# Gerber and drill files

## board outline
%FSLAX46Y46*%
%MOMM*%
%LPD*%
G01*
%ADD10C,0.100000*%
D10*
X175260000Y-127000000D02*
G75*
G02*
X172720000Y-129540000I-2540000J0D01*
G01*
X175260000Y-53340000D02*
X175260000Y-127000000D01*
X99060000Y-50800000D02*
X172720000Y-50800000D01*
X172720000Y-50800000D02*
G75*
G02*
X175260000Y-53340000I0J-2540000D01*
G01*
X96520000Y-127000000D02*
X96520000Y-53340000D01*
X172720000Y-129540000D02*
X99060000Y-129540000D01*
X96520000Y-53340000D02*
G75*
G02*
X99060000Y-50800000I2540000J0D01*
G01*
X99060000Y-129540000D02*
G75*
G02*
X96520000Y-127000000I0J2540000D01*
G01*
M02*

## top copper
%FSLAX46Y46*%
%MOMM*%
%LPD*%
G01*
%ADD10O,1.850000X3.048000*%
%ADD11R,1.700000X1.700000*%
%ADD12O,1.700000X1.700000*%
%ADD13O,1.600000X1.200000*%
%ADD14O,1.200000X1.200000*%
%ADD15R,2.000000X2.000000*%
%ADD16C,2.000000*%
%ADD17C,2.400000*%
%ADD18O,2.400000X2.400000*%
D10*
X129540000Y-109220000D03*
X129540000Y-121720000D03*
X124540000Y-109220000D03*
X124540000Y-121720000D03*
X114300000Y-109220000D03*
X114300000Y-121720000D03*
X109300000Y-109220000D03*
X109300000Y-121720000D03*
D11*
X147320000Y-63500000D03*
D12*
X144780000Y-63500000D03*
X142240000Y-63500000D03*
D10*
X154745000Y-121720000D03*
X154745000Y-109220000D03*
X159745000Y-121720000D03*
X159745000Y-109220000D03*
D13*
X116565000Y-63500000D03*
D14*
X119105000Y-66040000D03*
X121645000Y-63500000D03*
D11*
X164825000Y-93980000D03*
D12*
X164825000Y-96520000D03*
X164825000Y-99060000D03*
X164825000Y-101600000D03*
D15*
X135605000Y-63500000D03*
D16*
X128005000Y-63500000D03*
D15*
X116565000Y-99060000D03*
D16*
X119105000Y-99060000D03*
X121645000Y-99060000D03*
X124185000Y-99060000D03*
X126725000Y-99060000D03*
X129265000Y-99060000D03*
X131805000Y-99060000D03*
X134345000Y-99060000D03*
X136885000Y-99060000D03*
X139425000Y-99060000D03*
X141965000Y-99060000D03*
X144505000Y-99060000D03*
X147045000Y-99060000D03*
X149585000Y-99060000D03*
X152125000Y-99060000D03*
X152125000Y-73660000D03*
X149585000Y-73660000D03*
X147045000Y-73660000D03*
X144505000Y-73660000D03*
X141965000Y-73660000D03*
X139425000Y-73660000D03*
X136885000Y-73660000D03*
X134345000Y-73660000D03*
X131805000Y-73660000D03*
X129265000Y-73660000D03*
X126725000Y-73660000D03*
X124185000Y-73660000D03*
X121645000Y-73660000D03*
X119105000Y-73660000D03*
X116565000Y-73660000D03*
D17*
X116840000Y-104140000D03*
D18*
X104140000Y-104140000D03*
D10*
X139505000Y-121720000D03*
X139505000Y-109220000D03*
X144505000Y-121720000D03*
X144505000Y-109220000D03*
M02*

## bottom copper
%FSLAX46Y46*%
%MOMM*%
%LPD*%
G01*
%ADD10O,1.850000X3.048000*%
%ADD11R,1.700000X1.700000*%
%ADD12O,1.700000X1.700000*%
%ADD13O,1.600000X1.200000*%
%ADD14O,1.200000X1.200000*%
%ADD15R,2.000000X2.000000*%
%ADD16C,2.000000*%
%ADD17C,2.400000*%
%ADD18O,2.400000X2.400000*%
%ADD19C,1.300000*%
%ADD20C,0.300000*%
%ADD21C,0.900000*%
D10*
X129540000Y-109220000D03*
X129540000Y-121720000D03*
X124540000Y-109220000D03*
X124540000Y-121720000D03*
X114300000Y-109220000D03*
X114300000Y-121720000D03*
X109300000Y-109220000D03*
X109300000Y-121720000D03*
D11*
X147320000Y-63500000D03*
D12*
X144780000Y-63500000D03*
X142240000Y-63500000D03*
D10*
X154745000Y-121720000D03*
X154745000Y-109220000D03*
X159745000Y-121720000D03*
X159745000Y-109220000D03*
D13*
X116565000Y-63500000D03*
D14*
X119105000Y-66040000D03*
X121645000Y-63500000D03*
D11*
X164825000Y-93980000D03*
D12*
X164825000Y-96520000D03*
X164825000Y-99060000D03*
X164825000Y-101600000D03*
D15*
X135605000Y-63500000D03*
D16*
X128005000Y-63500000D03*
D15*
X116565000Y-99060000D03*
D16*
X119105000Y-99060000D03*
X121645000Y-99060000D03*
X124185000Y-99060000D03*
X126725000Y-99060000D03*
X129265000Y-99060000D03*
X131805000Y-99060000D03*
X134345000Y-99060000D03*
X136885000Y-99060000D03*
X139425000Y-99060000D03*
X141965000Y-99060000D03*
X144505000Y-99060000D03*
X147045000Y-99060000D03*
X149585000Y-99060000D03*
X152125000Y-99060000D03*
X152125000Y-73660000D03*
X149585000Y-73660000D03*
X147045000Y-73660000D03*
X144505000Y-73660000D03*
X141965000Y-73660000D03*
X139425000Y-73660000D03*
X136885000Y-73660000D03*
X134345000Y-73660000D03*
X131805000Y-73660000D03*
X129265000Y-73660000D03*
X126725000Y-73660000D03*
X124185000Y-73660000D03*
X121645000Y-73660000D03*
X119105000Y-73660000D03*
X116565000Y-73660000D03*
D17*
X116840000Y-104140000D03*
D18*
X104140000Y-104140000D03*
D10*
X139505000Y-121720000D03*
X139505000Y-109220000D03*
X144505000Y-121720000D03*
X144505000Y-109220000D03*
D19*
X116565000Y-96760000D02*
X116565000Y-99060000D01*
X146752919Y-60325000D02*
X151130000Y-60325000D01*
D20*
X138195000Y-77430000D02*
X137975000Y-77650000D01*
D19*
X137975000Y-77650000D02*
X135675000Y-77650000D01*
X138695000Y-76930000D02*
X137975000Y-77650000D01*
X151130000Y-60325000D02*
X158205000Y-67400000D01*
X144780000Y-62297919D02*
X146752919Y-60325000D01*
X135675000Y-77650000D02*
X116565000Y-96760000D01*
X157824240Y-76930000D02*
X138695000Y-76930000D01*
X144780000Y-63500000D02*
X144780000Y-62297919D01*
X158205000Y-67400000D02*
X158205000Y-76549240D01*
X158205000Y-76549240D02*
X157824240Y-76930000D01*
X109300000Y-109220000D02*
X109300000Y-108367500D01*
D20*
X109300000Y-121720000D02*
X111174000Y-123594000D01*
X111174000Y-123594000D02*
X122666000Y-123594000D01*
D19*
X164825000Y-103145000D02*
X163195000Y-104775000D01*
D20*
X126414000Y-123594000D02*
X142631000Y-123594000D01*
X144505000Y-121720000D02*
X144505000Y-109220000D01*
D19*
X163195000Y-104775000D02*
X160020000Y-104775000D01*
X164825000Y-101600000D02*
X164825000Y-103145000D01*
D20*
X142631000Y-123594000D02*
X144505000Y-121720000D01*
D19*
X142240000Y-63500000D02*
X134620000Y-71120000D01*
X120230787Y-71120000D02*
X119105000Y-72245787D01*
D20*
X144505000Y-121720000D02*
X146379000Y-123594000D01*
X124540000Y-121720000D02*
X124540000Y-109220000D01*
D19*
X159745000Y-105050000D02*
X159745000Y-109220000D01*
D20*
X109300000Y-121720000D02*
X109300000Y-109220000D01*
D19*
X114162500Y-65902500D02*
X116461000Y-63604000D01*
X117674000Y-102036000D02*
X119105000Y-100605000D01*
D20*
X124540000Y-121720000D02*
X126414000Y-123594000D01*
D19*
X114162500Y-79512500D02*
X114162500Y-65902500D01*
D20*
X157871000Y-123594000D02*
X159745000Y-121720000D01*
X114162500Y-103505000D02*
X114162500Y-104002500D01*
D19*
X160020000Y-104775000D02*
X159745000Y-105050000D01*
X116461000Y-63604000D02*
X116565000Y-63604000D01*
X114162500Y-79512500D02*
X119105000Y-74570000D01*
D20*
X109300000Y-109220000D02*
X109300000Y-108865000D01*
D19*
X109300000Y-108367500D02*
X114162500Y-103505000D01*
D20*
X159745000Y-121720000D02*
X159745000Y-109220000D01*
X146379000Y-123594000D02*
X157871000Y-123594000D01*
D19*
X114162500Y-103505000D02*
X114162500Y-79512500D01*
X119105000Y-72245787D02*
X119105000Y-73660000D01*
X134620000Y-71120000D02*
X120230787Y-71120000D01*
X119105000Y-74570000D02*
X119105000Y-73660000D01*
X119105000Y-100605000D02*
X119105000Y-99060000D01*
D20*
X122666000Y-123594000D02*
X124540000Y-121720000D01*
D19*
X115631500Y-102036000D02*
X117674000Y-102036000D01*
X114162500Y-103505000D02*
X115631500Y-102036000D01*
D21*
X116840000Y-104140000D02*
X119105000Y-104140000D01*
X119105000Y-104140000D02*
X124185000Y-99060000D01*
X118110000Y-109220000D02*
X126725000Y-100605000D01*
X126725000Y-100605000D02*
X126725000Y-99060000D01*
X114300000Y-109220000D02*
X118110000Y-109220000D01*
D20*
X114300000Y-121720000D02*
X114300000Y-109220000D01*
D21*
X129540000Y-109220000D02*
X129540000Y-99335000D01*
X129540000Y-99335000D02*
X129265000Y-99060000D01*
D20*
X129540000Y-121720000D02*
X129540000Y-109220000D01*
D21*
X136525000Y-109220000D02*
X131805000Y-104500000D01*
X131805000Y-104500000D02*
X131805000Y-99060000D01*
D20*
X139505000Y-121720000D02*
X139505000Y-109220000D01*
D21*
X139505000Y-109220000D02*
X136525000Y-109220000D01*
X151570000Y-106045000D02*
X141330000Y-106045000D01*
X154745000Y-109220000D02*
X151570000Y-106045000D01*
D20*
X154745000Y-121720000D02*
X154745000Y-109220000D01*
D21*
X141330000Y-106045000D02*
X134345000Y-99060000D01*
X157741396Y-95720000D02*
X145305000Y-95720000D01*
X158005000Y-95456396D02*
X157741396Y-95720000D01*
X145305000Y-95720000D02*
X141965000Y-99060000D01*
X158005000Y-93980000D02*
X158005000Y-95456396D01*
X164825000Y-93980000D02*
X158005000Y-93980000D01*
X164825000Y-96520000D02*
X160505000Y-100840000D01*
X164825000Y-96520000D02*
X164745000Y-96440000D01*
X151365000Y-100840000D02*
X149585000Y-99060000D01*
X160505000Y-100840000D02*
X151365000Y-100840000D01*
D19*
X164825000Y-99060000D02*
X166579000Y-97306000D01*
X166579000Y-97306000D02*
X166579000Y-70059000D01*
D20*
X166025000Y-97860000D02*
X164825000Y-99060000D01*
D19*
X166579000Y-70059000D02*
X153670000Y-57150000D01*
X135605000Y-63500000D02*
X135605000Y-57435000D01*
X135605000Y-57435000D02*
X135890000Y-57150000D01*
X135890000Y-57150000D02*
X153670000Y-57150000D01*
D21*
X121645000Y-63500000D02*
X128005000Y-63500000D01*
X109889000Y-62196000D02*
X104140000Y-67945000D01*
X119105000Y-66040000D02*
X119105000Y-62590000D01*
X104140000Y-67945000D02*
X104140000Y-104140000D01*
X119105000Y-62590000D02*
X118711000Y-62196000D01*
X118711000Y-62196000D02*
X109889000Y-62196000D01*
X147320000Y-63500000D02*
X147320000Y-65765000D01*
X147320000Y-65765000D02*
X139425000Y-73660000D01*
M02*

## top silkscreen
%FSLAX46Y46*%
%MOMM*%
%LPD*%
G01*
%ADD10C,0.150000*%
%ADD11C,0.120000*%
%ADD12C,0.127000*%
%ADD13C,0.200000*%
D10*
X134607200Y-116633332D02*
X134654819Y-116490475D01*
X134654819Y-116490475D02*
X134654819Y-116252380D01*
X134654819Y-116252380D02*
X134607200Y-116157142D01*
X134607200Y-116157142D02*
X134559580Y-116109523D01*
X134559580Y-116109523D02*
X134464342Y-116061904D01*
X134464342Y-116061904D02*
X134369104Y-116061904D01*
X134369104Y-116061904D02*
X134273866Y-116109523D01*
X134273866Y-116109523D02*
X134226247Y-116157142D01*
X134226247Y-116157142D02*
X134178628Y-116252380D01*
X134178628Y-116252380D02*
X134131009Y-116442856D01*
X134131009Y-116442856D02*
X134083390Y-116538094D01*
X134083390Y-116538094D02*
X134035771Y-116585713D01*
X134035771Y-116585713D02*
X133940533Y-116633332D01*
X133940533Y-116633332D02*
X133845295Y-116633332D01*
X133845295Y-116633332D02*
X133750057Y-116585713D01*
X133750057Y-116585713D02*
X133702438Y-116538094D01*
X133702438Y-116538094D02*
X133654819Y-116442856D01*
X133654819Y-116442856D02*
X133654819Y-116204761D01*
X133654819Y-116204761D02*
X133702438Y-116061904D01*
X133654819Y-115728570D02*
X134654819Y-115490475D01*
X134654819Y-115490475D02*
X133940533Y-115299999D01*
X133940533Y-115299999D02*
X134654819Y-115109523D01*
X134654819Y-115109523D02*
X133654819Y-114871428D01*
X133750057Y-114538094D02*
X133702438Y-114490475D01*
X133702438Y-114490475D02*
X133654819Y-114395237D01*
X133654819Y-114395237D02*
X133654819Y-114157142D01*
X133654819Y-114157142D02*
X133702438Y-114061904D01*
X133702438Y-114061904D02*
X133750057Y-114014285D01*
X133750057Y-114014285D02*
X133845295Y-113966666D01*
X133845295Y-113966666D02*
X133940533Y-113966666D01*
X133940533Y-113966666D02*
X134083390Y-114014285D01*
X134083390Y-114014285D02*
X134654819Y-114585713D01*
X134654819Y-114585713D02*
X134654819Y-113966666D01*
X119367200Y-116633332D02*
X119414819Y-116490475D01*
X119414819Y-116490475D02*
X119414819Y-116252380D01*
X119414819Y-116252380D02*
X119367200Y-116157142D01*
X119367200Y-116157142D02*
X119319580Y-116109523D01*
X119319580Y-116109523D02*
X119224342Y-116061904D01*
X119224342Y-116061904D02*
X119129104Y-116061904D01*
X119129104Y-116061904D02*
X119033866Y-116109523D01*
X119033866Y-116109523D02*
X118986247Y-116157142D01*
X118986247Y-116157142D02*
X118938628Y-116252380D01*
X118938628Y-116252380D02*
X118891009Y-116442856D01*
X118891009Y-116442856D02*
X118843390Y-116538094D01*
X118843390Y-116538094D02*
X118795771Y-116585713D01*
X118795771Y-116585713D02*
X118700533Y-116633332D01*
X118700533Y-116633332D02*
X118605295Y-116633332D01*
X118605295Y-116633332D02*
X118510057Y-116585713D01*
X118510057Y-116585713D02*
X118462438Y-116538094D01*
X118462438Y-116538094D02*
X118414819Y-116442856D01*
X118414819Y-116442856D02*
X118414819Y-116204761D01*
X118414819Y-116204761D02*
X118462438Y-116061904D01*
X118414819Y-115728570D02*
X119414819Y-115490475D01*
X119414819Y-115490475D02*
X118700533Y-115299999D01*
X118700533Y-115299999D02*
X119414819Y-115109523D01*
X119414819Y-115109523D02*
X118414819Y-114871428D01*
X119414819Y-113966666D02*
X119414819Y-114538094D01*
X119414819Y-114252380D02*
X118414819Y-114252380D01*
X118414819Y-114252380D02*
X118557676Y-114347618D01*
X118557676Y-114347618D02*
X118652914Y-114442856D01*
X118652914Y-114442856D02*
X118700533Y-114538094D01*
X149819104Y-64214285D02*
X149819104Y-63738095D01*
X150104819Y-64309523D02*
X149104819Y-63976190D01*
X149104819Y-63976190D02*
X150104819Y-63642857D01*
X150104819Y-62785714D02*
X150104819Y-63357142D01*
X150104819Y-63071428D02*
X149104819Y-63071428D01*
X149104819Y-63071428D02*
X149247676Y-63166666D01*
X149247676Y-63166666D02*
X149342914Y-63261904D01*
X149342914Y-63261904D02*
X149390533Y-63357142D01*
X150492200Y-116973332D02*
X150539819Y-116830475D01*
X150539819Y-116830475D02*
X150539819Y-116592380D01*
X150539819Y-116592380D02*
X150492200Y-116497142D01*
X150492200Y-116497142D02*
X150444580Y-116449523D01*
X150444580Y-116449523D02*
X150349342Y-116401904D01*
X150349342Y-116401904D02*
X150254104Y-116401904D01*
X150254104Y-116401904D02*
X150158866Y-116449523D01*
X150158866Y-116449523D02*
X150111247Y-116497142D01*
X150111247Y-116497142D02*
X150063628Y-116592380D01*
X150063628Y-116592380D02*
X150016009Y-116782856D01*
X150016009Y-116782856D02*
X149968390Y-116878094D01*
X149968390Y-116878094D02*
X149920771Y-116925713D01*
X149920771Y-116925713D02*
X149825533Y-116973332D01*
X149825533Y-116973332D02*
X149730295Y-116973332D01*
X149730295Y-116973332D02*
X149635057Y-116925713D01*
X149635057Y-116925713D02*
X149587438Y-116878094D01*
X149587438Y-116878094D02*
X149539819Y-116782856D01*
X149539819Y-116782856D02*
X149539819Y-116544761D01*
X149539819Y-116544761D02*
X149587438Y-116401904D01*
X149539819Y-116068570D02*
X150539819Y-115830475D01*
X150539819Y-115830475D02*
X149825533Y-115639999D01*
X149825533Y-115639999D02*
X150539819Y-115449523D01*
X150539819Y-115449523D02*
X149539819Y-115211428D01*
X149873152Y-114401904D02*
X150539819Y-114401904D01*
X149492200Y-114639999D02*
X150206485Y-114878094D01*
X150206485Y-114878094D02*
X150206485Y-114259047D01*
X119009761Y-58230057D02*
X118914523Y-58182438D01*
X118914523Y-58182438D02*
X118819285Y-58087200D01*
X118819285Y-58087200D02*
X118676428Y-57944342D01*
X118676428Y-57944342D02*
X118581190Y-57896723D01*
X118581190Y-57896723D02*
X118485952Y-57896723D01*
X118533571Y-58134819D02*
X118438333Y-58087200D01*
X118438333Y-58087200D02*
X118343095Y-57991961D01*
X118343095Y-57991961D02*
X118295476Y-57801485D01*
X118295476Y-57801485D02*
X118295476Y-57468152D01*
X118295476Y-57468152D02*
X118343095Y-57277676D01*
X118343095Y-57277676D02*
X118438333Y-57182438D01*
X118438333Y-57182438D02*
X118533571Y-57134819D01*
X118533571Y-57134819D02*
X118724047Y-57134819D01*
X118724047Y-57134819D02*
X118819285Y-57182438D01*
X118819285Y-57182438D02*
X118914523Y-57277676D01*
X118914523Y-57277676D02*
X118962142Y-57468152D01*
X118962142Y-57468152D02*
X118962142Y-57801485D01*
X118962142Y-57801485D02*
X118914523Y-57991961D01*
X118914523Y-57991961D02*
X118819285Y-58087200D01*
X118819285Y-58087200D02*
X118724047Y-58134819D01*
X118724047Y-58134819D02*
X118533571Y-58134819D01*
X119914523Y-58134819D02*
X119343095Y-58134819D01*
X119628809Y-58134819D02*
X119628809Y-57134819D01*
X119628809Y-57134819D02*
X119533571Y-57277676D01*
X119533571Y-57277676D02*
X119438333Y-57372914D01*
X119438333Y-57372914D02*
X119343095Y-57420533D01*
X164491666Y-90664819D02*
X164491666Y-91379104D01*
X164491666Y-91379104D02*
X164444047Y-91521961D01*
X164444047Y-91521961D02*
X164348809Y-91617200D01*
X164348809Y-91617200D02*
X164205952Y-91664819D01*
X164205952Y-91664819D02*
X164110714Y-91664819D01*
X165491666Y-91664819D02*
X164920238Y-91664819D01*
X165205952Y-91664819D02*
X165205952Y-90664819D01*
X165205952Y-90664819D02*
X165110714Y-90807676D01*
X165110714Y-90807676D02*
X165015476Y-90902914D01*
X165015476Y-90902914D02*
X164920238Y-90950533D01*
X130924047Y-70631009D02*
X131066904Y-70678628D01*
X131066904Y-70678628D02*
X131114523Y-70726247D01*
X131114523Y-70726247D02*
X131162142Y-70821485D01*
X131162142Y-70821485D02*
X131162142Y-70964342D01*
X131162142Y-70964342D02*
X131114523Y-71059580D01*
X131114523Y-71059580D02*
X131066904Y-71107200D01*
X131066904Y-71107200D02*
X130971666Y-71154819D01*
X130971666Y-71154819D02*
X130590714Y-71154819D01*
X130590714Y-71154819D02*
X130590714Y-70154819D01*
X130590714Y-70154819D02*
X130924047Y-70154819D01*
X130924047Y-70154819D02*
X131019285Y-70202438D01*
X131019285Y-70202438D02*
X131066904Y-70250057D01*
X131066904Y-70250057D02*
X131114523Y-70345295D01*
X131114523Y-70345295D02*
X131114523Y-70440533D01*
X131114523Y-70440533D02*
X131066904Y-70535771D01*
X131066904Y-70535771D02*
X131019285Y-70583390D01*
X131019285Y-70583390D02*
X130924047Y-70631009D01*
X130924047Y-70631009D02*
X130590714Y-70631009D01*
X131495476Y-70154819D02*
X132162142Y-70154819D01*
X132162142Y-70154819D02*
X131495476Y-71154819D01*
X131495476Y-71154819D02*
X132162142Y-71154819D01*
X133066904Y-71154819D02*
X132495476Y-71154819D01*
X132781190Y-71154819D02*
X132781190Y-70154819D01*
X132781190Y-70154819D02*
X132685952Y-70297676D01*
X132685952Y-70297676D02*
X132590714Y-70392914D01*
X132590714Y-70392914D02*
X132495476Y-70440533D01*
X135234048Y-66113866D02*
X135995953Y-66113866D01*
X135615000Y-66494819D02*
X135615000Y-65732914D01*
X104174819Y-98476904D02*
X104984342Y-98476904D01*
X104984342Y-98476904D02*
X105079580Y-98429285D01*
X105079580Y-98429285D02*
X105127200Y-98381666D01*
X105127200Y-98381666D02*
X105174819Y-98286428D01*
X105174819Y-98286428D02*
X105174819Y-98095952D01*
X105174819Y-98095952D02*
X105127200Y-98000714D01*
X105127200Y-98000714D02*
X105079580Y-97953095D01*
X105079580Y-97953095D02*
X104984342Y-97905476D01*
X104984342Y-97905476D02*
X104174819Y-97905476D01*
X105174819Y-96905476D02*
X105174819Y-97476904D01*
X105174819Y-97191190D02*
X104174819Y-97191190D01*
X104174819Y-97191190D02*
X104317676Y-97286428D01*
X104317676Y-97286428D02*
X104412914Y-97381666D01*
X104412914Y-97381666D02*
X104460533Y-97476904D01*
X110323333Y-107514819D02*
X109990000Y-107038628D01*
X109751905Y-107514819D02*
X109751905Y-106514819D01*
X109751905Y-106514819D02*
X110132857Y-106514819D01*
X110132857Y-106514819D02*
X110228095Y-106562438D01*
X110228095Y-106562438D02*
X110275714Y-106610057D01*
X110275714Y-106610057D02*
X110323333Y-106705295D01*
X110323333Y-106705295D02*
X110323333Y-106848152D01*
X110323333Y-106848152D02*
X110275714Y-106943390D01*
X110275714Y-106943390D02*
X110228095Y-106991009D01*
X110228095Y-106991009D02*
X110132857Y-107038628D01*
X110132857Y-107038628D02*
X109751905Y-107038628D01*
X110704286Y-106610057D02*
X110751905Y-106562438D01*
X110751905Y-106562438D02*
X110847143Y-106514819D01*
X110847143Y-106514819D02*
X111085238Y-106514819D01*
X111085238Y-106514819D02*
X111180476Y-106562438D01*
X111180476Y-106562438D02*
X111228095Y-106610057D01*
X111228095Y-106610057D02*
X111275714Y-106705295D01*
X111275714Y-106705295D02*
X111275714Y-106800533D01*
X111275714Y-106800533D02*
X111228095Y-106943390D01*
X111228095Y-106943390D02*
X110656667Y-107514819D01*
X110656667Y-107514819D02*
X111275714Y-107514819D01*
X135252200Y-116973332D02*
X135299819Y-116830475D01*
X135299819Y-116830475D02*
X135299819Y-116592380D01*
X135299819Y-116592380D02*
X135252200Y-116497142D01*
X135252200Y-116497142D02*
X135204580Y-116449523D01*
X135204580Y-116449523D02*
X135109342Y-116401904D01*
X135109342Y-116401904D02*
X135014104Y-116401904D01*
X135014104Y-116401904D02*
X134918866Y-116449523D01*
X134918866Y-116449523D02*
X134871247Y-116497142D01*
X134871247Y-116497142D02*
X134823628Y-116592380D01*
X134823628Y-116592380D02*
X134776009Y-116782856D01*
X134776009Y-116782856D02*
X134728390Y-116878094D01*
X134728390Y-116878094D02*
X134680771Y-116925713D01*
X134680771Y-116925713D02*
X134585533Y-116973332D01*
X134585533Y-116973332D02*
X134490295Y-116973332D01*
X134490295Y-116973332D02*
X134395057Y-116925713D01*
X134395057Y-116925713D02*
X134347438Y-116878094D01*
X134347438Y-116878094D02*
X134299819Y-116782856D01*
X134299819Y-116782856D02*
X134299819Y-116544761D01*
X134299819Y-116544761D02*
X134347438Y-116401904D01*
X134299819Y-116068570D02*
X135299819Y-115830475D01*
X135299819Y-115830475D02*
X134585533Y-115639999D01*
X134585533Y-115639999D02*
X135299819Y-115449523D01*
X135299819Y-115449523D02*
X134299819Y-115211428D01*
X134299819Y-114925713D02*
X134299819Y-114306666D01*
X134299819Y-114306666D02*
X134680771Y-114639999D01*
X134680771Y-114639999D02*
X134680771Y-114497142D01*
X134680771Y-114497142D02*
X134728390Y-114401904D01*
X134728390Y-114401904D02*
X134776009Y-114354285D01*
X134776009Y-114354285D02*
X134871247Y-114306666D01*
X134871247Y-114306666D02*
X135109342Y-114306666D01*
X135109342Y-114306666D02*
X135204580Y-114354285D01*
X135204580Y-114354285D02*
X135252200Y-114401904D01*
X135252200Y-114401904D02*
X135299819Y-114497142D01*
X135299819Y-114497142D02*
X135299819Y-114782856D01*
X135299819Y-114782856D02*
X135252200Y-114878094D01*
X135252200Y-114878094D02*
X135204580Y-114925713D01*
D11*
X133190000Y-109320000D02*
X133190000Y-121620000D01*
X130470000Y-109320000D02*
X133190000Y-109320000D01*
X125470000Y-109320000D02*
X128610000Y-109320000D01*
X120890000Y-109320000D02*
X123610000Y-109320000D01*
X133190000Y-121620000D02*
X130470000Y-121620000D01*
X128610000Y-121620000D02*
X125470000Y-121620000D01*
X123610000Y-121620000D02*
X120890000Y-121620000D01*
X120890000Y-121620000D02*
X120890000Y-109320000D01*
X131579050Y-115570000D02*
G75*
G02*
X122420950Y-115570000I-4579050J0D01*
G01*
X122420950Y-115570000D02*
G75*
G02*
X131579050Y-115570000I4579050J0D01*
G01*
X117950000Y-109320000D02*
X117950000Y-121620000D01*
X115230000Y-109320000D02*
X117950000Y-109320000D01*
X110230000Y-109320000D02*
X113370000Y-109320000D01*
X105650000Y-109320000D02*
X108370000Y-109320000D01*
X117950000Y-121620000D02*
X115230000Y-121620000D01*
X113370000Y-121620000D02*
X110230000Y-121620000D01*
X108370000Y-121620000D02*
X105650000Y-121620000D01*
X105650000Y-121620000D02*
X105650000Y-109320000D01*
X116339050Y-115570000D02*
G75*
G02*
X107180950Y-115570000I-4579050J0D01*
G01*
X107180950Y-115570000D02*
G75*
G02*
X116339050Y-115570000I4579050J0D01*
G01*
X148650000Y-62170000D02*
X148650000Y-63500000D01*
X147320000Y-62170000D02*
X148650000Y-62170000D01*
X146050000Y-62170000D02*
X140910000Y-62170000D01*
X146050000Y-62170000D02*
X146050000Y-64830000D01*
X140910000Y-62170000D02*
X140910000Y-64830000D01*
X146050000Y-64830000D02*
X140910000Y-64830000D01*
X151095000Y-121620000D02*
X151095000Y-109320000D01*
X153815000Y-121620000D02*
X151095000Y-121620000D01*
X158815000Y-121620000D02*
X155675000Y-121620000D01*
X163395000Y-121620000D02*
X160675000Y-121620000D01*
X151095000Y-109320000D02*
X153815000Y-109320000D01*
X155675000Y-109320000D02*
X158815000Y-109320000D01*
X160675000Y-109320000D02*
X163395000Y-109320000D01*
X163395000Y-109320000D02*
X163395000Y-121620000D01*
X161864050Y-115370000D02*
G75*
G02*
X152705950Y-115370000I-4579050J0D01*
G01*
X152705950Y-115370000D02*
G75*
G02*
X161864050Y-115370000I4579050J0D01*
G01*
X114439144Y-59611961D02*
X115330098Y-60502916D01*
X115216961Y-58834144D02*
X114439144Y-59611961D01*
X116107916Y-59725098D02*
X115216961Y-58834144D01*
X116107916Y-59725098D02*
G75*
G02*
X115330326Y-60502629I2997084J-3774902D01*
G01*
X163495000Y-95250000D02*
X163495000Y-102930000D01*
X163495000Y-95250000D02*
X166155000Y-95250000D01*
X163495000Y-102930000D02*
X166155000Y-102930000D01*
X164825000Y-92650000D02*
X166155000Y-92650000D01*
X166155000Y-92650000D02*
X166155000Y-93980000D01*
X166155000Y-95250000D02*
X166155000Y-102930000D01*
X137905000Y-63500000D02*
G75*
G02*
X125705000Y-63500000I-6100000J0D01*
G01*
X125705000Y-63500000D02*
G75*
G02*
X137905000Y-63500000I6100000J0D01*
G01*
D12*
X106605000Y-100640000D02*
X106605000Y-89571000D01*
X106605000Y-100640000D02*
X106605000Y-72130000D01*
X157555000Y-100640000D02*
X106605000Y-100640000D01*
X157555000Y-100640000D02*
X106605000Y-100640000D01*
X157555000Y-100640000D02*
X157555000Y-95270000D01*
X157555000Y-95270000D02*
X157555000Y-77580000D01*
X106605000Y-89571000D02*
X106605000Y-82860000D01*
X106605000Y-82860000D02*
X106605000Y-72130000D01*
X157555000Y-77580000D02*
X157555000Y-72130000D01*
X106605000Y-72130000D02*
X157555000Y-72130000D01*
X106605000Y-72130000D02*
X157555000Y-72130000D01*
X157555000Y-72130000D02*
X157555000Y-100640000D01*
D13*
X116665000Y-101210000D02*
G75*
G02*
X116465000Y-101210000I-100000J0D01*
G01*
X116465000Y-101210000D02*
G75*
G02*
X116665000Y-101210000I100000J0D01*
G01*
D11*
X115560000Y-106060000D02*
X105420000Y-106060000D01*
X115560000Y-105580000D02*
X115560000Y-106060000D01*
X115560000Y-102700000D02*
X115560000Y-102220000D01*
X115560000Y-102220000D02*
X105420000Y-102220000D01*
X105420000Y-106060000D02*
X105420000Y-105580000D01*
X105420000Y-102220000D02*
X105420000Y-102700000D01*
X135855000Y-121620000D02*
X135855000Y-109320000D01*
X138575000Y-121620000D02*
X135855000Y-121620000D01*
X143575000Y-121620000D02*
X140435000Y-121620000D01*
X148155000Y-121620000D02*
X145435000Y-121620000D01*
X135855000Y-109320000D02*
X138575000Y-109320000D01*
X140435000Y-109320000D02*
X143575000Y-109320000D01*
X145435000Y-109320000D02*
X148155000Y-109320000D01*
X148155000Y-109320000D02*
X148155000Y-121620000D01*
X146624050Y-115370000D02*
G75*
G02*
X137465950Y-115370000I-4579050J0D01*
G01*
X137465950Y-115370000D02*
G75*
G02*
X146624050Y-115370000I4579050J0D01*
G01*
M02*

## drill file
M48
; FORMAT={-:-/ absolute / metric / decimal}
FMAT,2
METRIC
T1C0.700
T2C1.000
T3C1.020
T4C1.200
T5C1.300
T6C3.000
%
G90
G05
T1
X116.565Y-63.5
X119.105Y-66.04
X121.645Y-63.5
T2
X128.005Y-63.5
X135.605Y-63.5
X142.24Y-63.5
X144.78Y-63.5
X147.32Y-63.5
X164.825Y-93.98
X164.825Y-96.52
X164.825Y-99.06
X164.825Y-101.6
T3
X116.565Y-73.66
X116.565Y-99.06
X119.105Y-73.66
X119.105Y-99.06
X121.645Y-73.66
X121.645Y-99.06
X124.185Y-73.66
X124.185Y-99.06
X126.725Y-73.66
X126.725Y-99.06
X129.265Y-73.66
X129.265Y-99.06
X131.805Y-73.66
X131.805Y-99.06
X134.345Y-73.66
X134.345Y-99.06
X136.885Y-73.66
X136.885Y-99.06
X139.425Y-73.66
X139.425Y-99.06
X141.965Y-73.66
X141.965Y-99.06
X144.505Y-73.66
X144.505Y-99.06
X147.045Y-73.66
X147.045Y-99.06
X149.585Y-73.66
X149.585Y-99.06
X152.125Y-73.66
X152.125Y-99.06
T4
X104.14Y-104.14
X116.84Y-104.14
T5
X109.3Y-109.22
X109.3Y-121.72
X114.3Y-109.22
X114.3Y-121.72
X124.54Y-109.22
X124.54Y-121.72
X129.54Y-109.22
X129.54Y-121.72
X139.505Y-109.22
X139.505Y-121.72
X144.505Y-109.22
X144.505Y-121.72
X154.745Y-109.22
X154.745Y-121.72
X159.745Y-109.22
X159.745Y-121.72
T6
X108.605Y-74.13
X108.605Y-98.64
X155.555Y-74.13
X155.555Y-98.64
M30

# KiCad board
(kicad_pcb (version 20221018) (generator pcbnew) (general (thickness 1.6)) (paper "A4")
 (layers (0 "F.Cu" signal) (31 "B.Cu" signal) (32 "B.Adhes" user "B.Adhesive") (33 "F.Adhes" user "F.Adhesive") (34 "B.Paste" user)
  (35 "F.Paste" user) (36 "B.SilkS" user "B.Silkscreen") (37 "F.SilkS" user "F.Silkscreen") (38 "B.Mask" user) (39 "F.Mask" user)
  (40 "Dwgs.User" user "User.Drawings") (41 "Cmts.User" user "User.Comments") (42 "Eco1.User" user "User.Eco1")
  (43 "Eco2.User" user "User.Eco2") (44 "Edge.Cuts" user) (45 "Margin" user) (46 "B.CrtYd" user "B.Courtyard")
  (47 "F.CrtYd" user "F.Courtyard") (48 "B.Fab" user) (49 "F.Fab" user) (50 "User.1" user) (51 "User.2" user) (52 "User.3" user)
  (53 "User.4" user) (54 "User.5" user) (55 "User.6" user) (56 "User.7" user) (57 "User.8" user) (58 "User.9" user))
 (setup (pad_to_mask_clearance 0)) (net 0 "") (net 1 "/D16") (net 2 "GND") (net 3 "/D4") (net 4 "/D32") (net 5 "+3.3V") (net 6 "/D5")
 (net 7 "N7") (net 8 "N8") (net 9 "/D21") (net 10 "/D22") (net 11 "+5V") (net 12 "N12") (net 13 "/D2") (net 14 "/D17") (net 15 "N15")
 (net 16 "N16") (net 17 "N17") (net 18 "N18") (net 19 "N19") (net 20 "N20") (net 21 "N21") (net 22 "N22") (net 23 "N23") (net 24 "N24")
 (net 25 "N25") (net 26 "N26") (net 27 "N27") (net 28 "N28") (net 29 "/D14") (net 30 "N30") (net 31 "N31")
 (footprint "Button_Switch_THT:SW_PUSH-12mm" (layer "F.Cu") (at 129.54 109.22 -90)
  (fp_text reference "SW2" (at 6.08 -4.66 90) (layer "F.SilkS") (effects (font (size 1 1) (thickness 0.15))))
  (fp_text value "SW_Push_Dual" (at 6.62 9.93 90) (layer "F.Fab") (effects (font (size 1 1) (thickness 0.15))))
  (fp_line (start 0.1 -3.65) (end 12.4 -3.65) (stroke (width 0.12) (type solid)) (layer "F.SilkS"))
  (fp_line (start 0.1 -0.93) (end 0.1 -3.65) (stroke (width 0.12) (type solid)) (layer "F.SilkS"))
  (fp_line (start 0.1 4.07) (end 0.1 0.93) (stroke (width 0.12) (type solid)) (layer "F.SilkS"))
  (fp_line (start 0.1 8.65) (end 0.1 5.93) (stroke (width 0.12) (type solid)) (layer "F.SilkS"))
  (fp_line (start 12.4 -3.65) (end 12.4 -0.93) (stroke (width 0.12) (type solid)) (layer "F.SilkS"))
  (fp_line (start 12.4 0.93) (end 12.4 4.07) (stroke (width 0.12) (type solid)) (layer "F.SilkS"))
  (fp_line (start 12.4 5.93) (end 12.4 8.65) (stroke (width 0.12) (type solid)) (layer "F.SilkS"))
  (fp_line (start 12.4 8.65) (end 0.1 8.65) (stroke (width 0.12) (type solid)) (layer "F.SilkS"))
  (fp_circle (center 6.35 2.54) (end 10.16 5.08) (stroke (width 0.12) (type solid)) (fill none) (layer "F.SilkS"))
  (pad "1" thru_hole oval (at 0 0 270) (size 3.048 1.85) (drill 1.3) (layers "*.Cu" "*.Mask") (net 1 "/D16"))
  (pad "1" thru_hole oval (at 12.5 0 270) (size 3.048 1.85) (drill 1.3) (layers "*.Cu" "*.Mask") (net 1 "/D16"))
  (pad "2" thru_hole oval (at 0 5 270) (size 3.048 1.85) (drill 1.3) (layers "*.Cu" "*.Mask") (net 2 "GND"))
  (pad "2" thru_hole oval (at 12.5 5 270) (size 3.048 1.85) (drill 1.3) (layers "*.Cu" "*.Mask") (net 2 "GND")))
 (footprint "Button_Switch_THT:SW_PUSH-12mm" (layer "F.Cu") (at 114.3 109.22 -90)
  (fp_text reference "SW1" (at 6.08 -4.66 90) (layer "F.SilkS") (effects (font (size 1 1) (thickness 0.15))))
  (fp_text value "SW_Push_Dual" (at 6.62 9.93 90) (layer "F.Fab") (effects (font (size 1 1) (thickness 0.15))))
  (fp_line (start 0.1 -3.65) (end 12.4 -3.65) (stroke (width 0.12) (type solid)) (layer "F.SilkS"))
  (fp_line (start 0.1 -0.93) (end 0.1 -3.65) (stroke (width 0.12) (type solid)) (layer "F.SilkS"))
  (fp_line (start 0.1 4.07) (end 0.1 0.93) (stroke (width 0.12) (type solid)) (layer "F.SilkS"))
  (fp_line (start 0.1 8.65) (end 0.1 5.93) (stroke (width 0.12) (type solid)) (layer "F.SilkS"))
  (fp_line (start 12.4 -3.65) (end 12.4 -0.93) (stroke (width 0.12) (type solid)) (layer "F.SilkS"))
  (fp_line (start 12.4 0.93) (end 12.4 4.07) (stroke (width 0.12) (type solid)) (layer "F.SilkS"))
  (fp_line (start 12.4 5.93) (end 12.4 8.65) (stroke (width 0.12) (type solid)) (layer "F.SilkS"))
  (fp_line (start 12.4 8.65) (end 0.1 8.65) (stroke (width 0.12) (type solid)) (layer "F.SilkS"))
  (fp_circle (center 6.35 2.54) (end 10.16 5.08) (stroke (width 0.12) (type solid)) (fill none) (layer "F.SilkS"))
  (pad "1" thru_hole oval (at 0 0 270) (size 3.048 1.85) (drill 1.3) (layers "*.Cu" "*.Mask") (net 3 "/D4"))
  (pad "1" thru_hole oval (at 12.5 0 270) (size 3.048 1.85) (drill 1.3) (layers "*.Cu" "*.Mask") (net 3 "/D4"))
  (pad "2" thru_hole oval (at 0 5 270) (size 3.048 1.85) (drill 1.3) (layers "*.Cu" "*.Mask") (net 2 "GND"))
  (pad "2" thru_hole oval (at 12.5 5 270) (size 3.048 1.85) (drill 1.3) (layers "*.Cu" "*.Mask") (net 2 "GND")))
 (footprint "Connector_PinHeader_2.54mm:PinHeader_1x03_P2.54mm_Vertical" (layer "F.Cu") (at 147.32 63.5 -90)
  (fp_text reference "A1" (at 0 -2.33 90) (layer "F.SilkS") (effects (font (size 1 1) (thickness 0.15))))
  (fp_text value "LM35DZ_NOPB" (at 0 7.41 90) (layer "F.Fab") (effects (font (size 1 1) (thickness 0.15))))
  (fp_line (start -1.33 -1.33) (end 0 -1.33) (stroke (width 0.12) (type solid)) (layer "F.SilkS"))
  (fp_line (start -1.33 0) (end -1.33 -1.33) (stroke (width 0.12) (type solid)) (layer "F.SilkS"))
  (fp_line (start -1.33 1.27) (end -1.33 6.41) (stroke (width 0.12) (type solid)) (layer "F.SilkS"))
  (fp_line (start -1.33 1.27) (end 1.33 1.27) (stroke (width 0.12) (type solid)) (layer "F.SilkS"))
  (fp_line (start -1.33 6.41) (end 1.33 6.41) (stroke (width 0.12) (type solid)) (layer "F.SilkS"))
  (fp_line (start 1.33 1.27) (end 1.33 6.41) (stroke (width 0.12) (type solid)) (layer "F.SilkS"))
  (pad "1" thru_hole rect (at 0 0 270) (size 1.7 1.7) (drill 1) (layers "*.Cu" "*.Mask") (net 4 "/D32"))
  (pad "2" thru_hole oval (at 0 2.54 270) (size 1.7 1.7) (drill 1) (layers "*.Cu" "*.Mask") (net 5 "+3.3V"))
  (pad "3" thru_hole oval (at 0 5.08 270) (size 1.7 1.7) (drill 1) (layers "*.Cu" "*.Mask") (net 2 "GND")))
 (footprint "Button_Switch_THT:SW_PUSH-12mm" (layer "F.Cu") (at 154.745 121.72 90)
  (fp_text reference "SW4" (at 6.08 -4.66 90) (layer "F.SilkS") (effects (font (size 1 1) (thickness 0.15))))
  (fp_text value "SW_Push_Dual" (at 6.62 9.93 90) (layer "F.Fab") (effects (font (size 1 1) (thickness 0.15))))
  (fp_line (start 0.1 -3.65) (end 12.4 -3.65) (stroke (width 0.12) (type solid)) (layer "F.SilkS"))
  (fp_line (start 0.1 -0.93) (end 0.1 -3.65) (stroke (width 0.12) (type solid)) (layer "F.SilkS"))
  (fp_line (start 0.1 4.07) (end 0.1 0.93) (stroke (width 0.12) (type solid)) (layer "F.SilkS"))
  (fp_line (start 0.1 8.65) (end 0.1 5.93) (stroke (width 0.12) (type solid)) (layer "F.SilkS"))
  (fp_line (start 12.4 -3.65) (end 12.4 -0.93) (stroke (width 0.12) (type solid)) (layer "F.SilkS"))
  (fp_line (start 12.4 0.93) (end 12.4 4.07) (stroke (width 0.12) (type solid)) (layer "F.SilkS"))
  (fp_line (start 12.4 5.93) (end 12.4 8.65) (stroke (width 0.12) (type solid)) (layer "F.SilkS"))
  (fp_line (start 12.4 8.65) (end 0.1 8.65) (stroke (width 0.12) (type solid)) (layer "F.SilkS"))
  (fp_circle (center 6.35 2.54) (end 10.16 5.08) (stroke (width 0.12) (type solid)) (fill none) (layer "F.SilkS"))
  (pad "1" thru_hole oval (at 0 0 90) (size 3.048 1.85) (drill 1.3) (layers "*.Cu" "*.Mask") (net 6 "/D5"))
  (pad "1" thru_hole oval (at 12.5 0 90) (size 3.048 1.85) (drill 1.3) (layers "*.Cu" "*.Mask") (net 6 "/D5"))
  (pad "2" thru_hole oval (at 0 5 90) (size 3.048 1.85) (drill 1.3) (layers "*.Cu" "*.Mask") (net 2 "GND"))
  (pad "2" thru_hole oval (at 12.5 5 90) (size 3.048 1.85) (drill 1.3) (layers "*.Cu" "*.Mask") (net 2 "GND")))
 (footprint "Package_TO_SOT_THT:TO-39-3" (layer "F.Cu") (at 116.565 63.5)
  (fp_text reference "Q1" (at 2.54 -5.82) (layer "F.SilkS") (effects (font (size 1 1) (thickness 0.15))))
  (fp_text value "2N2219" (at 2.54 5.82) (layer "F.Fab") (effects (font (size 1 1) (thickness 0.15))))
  (fp_line (start -2.125856 -3.888039) (end -1.234902 -2.997084) (stroke (width 0.12) (type solid)) (layer "F.SilkS"))
  (fp_line (start -1.348039 -4.665856) (end -2.125856 -3.888039) (stroke (width 0.12) (type solid)) (layer "F.SilkS"))
  (fp_line (start -0.457084 -3.774902) (end -1.348039 -4.665856) (stroke (width 0.12) (type solid)) (layer "F.SilkS"))
  (fp_arc (start -0.457084 -3.774902) (mid 5.948125 3.408384) (end -1.234674 -2.997371) (stroke (width 0.12) (type solid)) (layer "F.SilkS"))
  (pad "1" thru_hole oval (at 0 0) (size 1.6 1.2) (drill 0.7) (layers "*.Cu" "*.Mask") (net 2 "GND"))
  (pad "2" thru_hole oval (at 2.54 2.54) (size 1.2 1.2) (drill 0.7) (layers "*.Cu" "*.Mask") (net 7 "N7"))
  (pad "3" thru_hole oval (at 5.08 0) (size 1.2 1.2) (drill 0.7) (layers "*.Cu" "*.Mask") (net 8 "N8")))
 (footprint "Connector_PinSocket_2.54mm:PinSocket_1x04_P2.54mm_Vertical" (layer "F.Cu") (at 164.825 93.98)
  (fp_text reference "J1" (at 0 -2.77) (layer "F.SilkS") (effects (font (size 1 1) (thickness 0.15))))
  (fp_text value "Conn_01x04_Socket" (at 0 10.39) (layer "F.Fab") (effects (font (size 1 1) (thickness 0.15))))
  (fp_line (start -1.33 1.27) (end -1.33 8.95) (stroke (width 0.12) (type solid)) (layer "F.SilkS"))
  (fp_line (start -1.33 1.27) (end 1.33 1.27) (stroke (width 0.12) (type solid)) (layer "F.SilkS"))
  (fp_line (start -1.33 8.95) (end 1.33 8.95) (stroke (width 0.12) (type solid)) (layer "F.SilkS"))
  (fp_line (start 0 -1.33) (end 1.33 -1.33) (stroke (width 0.12) (type solid)) (layer "F.SilkS"))
  (fp_line (start 1.33 -1.33) (end 1.33 0) (stroke (width 0.12) (type solid)) (layer "F.SilkS"))
  (fp_line (start 1.33 1.27) (end 1.33 8.95) (stroke (width 0.12) (type solid)) (layer "F.SilkS"))
  (pad "1" thru_hole rect (at 0 0) (size 1.7 1.7) (drill 1) (layers "*.Cu" "*.Mask") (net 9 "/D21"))
  (pad "2" thru_hole oval (at 0 2.54) (size 1.7 1.7) (drill 1) (layers "*.Cu" "*.Mask") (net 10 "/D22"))
  (pad "3" thru_hole oval (at 0 5.08) (size 1.7 1.7) (drill 1) (layers "*.Cu" "*.Mask") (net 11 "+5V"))
  (pad "4" thru_hole oval (at 0 7.62) (size 1.7 1.7) (drill 1) (layers "*.Cu" "*.Mask") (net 2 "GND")))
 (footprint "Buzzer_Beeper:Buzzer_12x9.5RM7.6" (layer "F.Cu") (at 135.605 63.5 180)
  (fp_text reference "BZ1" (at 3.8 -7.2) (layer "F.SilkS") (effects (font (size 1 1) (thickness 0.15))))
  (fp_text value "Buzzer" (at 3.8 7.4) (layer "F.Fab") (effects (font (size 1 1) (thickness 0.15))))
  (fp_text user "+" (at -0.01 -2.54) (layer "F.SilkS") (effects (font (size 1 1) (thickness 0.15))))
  (fp_circle (center 3.8 0) (end 9.9 0) (stroke (width 0.12) (type solid)) (fill none) (layer "F.SilkS"))
  (pad "1" thru_hole rect (at 0 0 180) (size 2 2) (drill 1) (layers "*.Cu" "*.Mask") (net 11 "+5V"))
  (pad "2" thru_hole circle (at 7.6 0 180) (size 2 2) (drill 1) (layers "*.Cu" "*.Mask") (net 8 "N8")))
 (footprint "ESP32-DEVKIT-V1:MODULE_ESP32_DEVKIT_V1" (layer "F.Cu") (at 132.08 86.36 90)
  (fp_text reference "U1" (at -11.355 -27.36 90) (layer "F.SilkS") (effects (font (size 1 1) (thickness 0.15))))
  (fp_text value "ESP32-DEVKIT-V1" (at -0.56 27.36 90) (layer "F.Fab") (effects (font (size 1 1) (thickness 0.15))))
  (fp_line (start -14.28 -25.475) (end -3.211 -25.475) (stroke (width 0.127) (type solid)) (layer "F.SilkS"))
  (fp_line (start -14.28 -25.475) (end 14.23 -25.475) (stroke (width 0.127) (type solid)) (layer "F.SilkS"))
  (fp_line (start -14.28 25.475) (end -14.28 -25.475) (stroke (width 0.127) (type solid)) (layer "F.SilkS"))
  (fp_line (start -14.28 25.475) (end -14.28 -25.475) (stroke (width 0.127) (type solid)) (layer "F.SilkS"))
  (fp_line (start -14.28 25.475) (end -8.91 25.475) (stroke (width 0.127) (type solid)) (layer "F.SilkS"))
  (fp_line (start -8.91 25.475) (end 8.78 25.475) (stroke (width 0.127) (type solid)) (layer "F.SilkS"))
  (fp_line (start -3.211 -25.475) (end 3.5 -25.475) (stroke (width 0.127) (type solid)) (layer "F.SilkS"))
  (fp_line (start 3.5 -25.475) (end 14.23 -25.475) (stroke (width 0.127) (type solid)) (layer "F.SilkS"))
  (fp_line (start 8.78 25.475) (end 14.23 25.475) (stroke (width 0.127) (type solid)) (layer "F.SilkS"))
  (fp_line (start 14.23 -25.475) (end 14.23 25.475) (stroke (width 0.127) (type solid)) (layer "F.SilkS"))
  (fp_line (start 14.23 -25.475) (end 14.23 25.475) (stroke (width 0.127) (type solid)) (layer "F.SilkS"))
  (fp_line (start 14.23 25.475) (end -14.28 25.475) (stroke (width 0.127) (type solid)) (layer "F.SilkS"))
  (fp_circle (center -14.85 -15.515) (end -14.75 -15.515) (stroke (width 0.2) (type solid)) (fill none) (layer "F.SilkS"))
  (pad "" np_thru_hole circle (at -12.28 -23.475 90) (size 3 3) (drill 3) (layers "*.Cu" "*.Mask"))
  (pad "" np_thru_hole circle (at -12.28 23.475 90) (size 3 3) (drill 3) (layers "*.Cu" "*.Mask"))
  (pad "" np_thru_hole circle (at 12.23 -23.475 90) (size 3 3) (drill 3) (layers "*.Cu" "*.Mask"))
  (pad "" np_thru_hole circle (at 12.23 23.475 90) (size 3 3) (drill 3) (layers "*.Cu" "*.Mask"))
  (pad "1" thru_hole rect (at -12.7 -15.515 90) (size 2 2) (drill 1.02) (layers "*.Cu" "*.Mask") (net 5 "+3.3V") (solder_mask_margin 0.102))
  (pad "2" thru_hole circle (at -12.7 -12.975 90) (size 2 2) (drill 1.02) (layers "*.Cu" "*.Mask") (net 2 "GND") (solder_mask_margin 0.102))
  (pad "3" thru_hole circle (at -12.7 -10.435 90) (size 2 2) (drill 1.02) (layers "*.Cu" "*.Mask") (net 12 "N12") (solder_mask_margin 0.102))
  (pad "4" thru_hole circle (at -12.7 -7.895 90) (size 2 2) (drill 1.02) (layers "*.Cu" "*.Mask") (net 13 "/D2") (solder_mask_margin 0.102))
  (pad "5" thru_hole circle (at -12.7 -5.355 90) (size 2 2) (drill 1.02) (layers "*.Cu" "*.Mask") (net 3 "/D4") (solder_mask_margin 0.102))
  (pad "6" thru_hole circle (at -12.7 -2.815 90) (size 2 2) (drill 1.02) (layers "*.Cu" "*.Mask") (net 1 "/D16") (solder_mask_margin 0.102))
  (pad "7" thru_hole circle (at -12.7 -0.275 90) (size 2 2) (drill 1.02) (layers "*.Cu" "*.Mask") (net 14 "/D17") (solder_mask_margin 0.102))
  (pad "8" thru_hole circle (at -12.7 2.265 90) (size 2 2) (drill 1.02) (layers "*.Cu" "*.Mask") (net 6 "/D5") (solder_mask_margin 0.102))
  (pad "9" thru_hole circle (at -12.7 4.805 90) (size 2 2) (drill 1.02) (layers "*.Cu" "*.Mask") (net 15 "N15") (solder_mask_margin 0.102))
  (pad "10" thru_hole circle (at -12.7 7.345 90) (size 2 2) (drill 1.02) (layers "*.Cu" "*.Mask") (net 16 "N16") (solder_mask_margin 0.102))
  (pad "11" thru_hole circle (at -12.7 9.885 90) (size 2 2) (drill 1.02) (layers "*.Cu" "*.Mask") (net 9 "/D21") (solder_mask_margin 0.102))
  (pad "12" thru_hole circle (at -12.7 12.425 90) (size 2 2) (drill 1.02) (layers "*.Cu" "*.Mask") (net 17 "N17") (solder_mask_margin 0.102))
  (pad "13" thru_hole circle (at -12.7 14.965 90) (size 2 2) (drill 1.02) (layers "*.Cu" "*.Mask") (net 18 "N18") (solder_mask_margin 0.102))
  (pad "14" thru_hole circle (at -12.7 17.505 90) (size 2 2) (drill 1.02) (layers "*.Cu" "*.Mask") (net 10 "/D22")
   (solder_mask_margin 0.102))
  (pad "15" thru_hole circle (at -12.7 20.045 90) (size 2 2) (drill 1.02) (layers "*.Cu" "*.Mask") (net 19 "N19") (solder_mask_margin 0.102))
  (pad "16" thru_hole circle (at 12.7 20.045 90) (size 2 2) (drill 1.02) (layers "*.Cu" "*.Mask") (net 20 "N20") (solder_mask_margin 0.102))
  (pad "17" thru_hole circle (at 12.7 17.505 90) (size 2 2) (drill 1.02) (layers "*.Cu" "*.Mask") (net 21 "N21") (solder_mask_margin 0.102))
  (pad "18" thru_hole circle (at 12.7 14.965 90) (size 2 2) (drill 1.02) (layers "*.Cu" "*.Mask") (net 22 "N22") (solder_mask_margin 0.102))
  (pad "19" thru_hole circle (at 12.7 12.425 90) (size 2 2) (drill 1.02) (layers "*.Cu" "*.Mask") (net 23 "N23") (solder_mask_margin 0.102))
  (pad "20" thru_hole circle (at 12.7 9.885 90) (size 2 2) (drill 1.02) (layers "*.Cu" "*.Mask") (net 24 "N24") (solder_mask_margin 0.102))
  (pad "21" thru_hole circle (at 12.7 7.345 90) (size 2 2) (drill 1.02) (layers "*.Cu" "*.Mask") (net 4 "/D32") (solder_mask_margin 0.102))
  (pad "22" thru_hole circle (at 12.7 4.805 90) (size 2 2) (drill 1.02) (layers "*.Cu" "*.Mask") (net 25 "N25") (solder_mask_margin 0.102))
  (pad "23" thru_hole circle (at 12.7 2.265 90) (size 2 2) (drill 1.02) (layers "*.Cu" "*.Mask") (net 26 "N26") (solder_mask_margin 0.102))
  (pad "24" thru_hole circle (at 12.7 -0.275 90) (size 2 2) (drill 1.02) (layers "*.Cu" "*.Mask") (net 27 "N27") (solder_mask_margin 0.102))
  (pad "25" thru_hole circle (at 12.7 -2.815 90) (size 2 2) (drill 1.02) (layers "*.Cu" "*.Mask") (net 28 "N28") (solder_mask_margin 0.102))
  (pad "26" thru_hole circle (at 12.7 -5.355 90) (size 2 2) (drill 1.02) (layers "*.Cu" "*.Mask") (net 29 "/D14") (solder_mask_margin 0.102))
  (pad "27" thru_hole circle (at 12.7 -7.895 90) (size 2 2) (drill 1.02) (layers "*.Cu" "*.Mask") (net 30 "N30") (solder_mask_margin 0.102))
  (pad "28" thru_hole circle (at 12.7 -10.435 90) (size 2 2) (drill 1.02) (layers "*.Cu" "*.Mask") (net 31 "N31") (solder_mask_margin 0.102))
  (pad "29" thru_hole circle (at 12.7 -12.975 90) (size 2 2) (drill 1.02) (layers "*.Cu" "*.Mask") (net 2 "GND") (solder_mask_margin 0.102))
  (pad "30" thru_hole circle (at 12.7 -15.515 90) (size 2 2) (drill 1.02) (layers "*.Cu" "*.Mask") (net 11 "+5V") (solder_mask_margin 0.102))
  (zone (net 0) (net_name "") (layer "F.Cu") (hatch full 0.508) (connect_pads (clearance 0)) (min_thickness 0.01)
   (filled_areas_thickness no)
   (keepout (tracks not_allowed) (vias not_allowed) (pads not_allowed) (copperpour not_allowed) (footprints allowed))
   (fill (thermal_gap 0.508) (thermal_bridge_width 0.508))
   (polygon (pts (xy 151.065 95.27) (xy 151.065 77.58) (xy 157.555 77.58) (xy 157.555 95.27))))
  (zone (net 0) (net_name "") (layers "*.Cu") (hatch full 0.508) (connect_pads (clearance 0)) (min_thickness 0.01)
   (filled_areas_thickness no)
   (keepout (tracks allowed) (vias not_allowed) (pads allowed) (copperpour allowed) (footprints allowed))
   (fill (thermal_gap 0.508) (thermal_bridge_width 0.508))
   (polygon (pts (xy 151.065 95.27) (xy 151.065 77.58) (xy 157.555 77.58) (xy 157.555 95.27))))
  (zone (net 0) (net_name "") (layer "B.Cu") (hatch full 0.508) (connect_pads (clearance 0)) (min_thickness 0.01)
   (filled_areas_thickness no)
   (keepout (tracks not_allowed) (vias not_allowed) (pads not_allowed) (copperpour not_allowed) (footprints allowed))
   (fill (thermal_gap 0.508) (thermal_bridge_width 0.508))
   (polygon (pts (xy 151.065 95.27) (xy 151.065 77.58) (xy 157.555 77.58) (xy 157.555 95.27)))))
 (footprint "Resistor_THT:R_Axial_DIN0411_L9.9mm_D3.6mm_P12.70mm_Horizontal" (layer "F.Cu") (at 116.84 104.14 180)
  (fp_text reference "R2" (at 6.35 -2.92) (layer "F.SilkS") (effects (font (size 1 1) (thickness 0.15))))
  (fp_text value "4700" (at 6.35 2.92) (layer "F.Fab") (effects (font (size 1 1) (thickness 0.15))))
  (fp_line (start 1.28 -1.92) (end 11.42 -1.92) (stroke (width 0.12) (type solid)) (layer "F.SilkS"))
  (fp_line (start 1.28 -1.44) (end 1.28 -1.92) (stroke (width 0.12) (type solid)) (layer "F.SilkS"))
  (fp_line (start 1.28 1.44) (end 1.28 1.92) (stroke (width 0.12) (type solid)) (layer "F.SilkS"))
  (fp_line (start 1.28 1.92) (end 11.42 1.92) (stroke (width 0.12) (type solid)) (layer "F.SilkS"))
  (fp_line (start 11.42 -1.92) (end 11.42 -1.44) (stroke (width 0.12) (type solid)) (layer "F.SilkS"))
  (fp_line (start 11.42 1.92) (end 11.42 1.44) (stroke (width 0.12) (type solid)) (layer "F.SilkS"))
  (pad "1" thru_hole circle (at 0 0 180) (size 2.4 2.4) (drill 1.2) (layers "*.Cu" "*.Mask") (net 13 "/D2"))
  (pad "2" thru_hole oval (at 12.7 0 180) (size 2.4 2.4) (drill 1.2) (layers "*.Cu" "*.Mask") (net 7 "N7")))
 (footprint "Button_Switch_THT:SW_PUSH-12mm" (layer "F.Cu") (at 139.505 121.72 90)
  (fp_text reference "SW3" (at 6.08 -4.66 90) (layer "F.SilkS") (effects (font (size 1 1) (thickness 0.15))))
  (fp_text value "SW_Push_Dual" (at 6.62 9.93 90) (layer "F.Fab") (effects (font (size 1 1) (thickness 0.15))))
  (fp_line (start 0.1 -3.65) (end 12.4 -3.65) (stroke (width 0.12) (type solid)) (layer "F.SilkS"))
  (fp_line (start 0.1 -0.93) (end 0.1 -3.65) (stroke (width 0.12) (type solid)) (layer "F.SilkS"))
  (fp_line (start 0.1 4.07) (end 0.1 0.93) (stroke (width 0.12) (type solid)) (layer "F.SilkS"))
  (fp_line (start 0.1 8.65) (end 0.1 5.93) (stroke (width 0.12) (type solid)) (layer "F.SilkS"))
  (fp_line (start 12.4 -3.65) (end 12.4 -0.93) (stroke (width 0.12) (type solid)) (layer "F.SilkS"))
  (fp_line (start 12.4 0.93) (end 12.4 4.07) (stroke (width 0.12) (type solid)) (layer "F.SilkS"))
  (fp_line (start 12.4 5.93) (end 12.4 8.65) (stroke (width 0.12) (type solid)) (layer "F.SilkS"))
  (fp_line (start 12.4 8.65) (end 0.1 8.65) (stroke (width 0.12) (type solid)) (layer "F.SilkS"))
  (fp_circle (center 6.35 2.54) (end 10.16 5.08) (stroke (width 0.12) (type solid)) (fill none) (layer "F.SilkS"))
  (pad "1" thru_hole oval (at 0 0 90) (size 3.048 1.85) (drill 1.3) (layers "*.Cu" "*.Mask") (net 14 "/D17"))
  (pad "1" thru_hole oval (at 12.5 0 90) (size 3.048 1.85) (drill 1.3) (layers "*.Cu" "*.Mask") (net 14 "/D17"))
  (pad "2" thru_hole oval (at 0 5 90) (size 3.048 1.85) (drill 1.3) (layers "*.Cu" "*.Mask") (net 2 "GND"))
  (pad "2" thru_hole oval (at 12.5 5 90) (size 3.048 1.85) (drill 1.3) (layers "*.Cu" "*.Mask") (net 2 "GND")))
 (gr_arc (start 175.26 127) (mid 174.516051 128.796051) (end 172.72 129.54) (stroke (width 0.1) (type default)) (layer "Edge.Cuts"))
 (gr_line (start 175.26 53.34) (end 175.26 127) (stroke (width 0.1) (type default)) (layer "Edge.Cuts"))
 (gr_line (start 99.06 50.8) (end 172.72 50.8) (stroke (width 0.1) (type default)) (layer "Edge.Cuts"))
 (gr_arc (start 172.72 50.8) (mid 174.516051 51.543949) (end 175.26 53.34) (stroke (width 0.1) (type default)) (layer "Edge.Cuts"))
 (gr_line (start 96.52 127) (end 96.52 53.34) (stroke (width 0.1) (type default)) (layer "Edge.Cuts"))
 (gr_line (start 172.72 129.54) (end 99.06 129.54) (stroke (width 0.1) (type default)) (layer "Edge.Cuts"))
 (gr_arc (start 96.52 53.34) (mid 97.263949 51.543949) (end 99.06 50.8) (stroke (width 0.1) (type default)) (layer "Edge.Cuts"))
 (gr_arc (start 99.06 129.54) (mid 97.263949 128.796051) (end 96.52 127) (stroke (width 0.1) (type default)) (layer "Edge.Cuts"))
 (segment (start 116.565 96.76) (end 116.565 99.06) (width 1.3) (layer "B.Cu") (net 5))
 (segment (start 146.752919 60.325) (end 151.13 60.325) (width 1.3) (layer "B.Cu") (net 5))
 (segment (start 138.195 77.43) (end 137.975 77.65) (width 0.3) (layer "B.Cu") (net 5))
 (segment (start 137.975 77.65) (end 135.675 77.65) (width 1.3) (layer "B.Cu") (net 5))
 (segment (start 138.695 76.93) (end 137.975 77.65) (width 1.3) (layer "B.Cu") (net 5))
 (segment (start 151.13 60.325) (end 158.205 67.4) (width 1.3) (layer "B.Cu") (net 5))
 (segment (start 144.78 62.297919) (end 146.752919 60.325) (width 1.3) (layer "B.Cu") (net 5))
 (segment (start 135.675 77.65) (end 116.565 96.76) (width 1.3) (layer "B.Cu") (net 5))
 (segment (start 157.82424 76.93) (end 138.695 76.93) (width 1.3) (layer "B.Cu") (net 5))
 (segment (start 144.78 63.5) (end 144.78 62.297919) (width 1.3) (layer "B.Cu") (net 5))
 (segment (start 158.205 67.4) (end 158.205 76.54924) (width 1.3) (layer "B.Cu") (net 5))
 (segment (start 158.205 76.54924) (end 157.82424 76.93) (width 1.3) (layer "B.Cu") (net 5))
 (segment (start 109.3 109.22) (end 109.3 108.3675) (width 1.3) (layer "B.Cu") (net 2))
 (segment (start 109.3 121.72) (end 111.174 123.594) (width 0.3) (layer "B.Cu") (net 2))
 (segment (start 111.174 123.594) (end 122.666 123.594) (width 0.3) (layer "B.Cu") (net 2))
 (segment (start 164.825 103.145) (end 163.195 104.775) (width 1.3) (layer "B.Cu") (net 2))
 (segment (start 126.414 123.594) (end 142.631 123.594) (width 0.3) (layer "B.Cu") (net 2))
 (segment (start 144.505 121.72) (end 144.505 109.22) (width 0.3) (layer "B.Cu") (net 2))
 (segment (start 163.195 104.775) (end 160.02 104.775) (width 1.3) (layer "B.Cu") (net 2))
 (segment (start 164.825 101.6) (end 164.825 103.145) (width 1.3) (layer "B.Cu") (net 2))
 (segment (start 142.631 123.594) (end 144.505 121.72) (width 0.3) (layer "B.Cu") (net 2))
 (segment (start 142.24 63.5) (end 134.62 71.12) (width 1.3) (layer "B.Cu") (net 2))
 (segment (start 120.230787 71.12) (end 119.105 72.245787) (width 1.3) (layer "B.Cu") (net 2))
 (segment (start 144.505 121.72) (end 146.379 123.594) (width 0.3) (layer "B.Cu") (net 2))
 (segment (start 124.54 121.72) (end 124.54 109.22) (width 0.3) (layer "B.Cu") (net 2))
 (segment (start 159.745 105.05) (end 159.745 109.22) (width 1.3) (layer "B.Cu") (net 2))
 (segment (start 109.3 121.72) (end 109.3 109.22) (width 0.3) (layer "B.Cu") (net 2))
 (segment (start 114.1625 65.9025) (end 116.461 63.604) (width 1.3) (layer "B.Cu") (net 2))
 (segment (start 117.674 102.036) (end 119.105 100.605) (width 1.3) (layer "B.Cu") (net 2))
 (segment (start 124.54 121.72) (end 126.414 123.594) (width 0.3) (layer "B.Cu") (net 2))
 (segment (start 114.1625 79.5125) (end 114.1625 65.9025) (width 1.3) (layer "B.Cu") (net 2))
 (segment (start 157.871 123.594) (end 159.745 121.72) (width 0.3) (layer "B.Cu") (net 2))
 (segment (start 114.1625 103.505) (end 114.1625 104.0025) (width 0.3) (layer "B.Cu") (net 2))
 (segment (start 160.02 104.775) (end 159.745 105.05) (width 1.3) (layer "B.Cu") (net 2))
 (segment (start 116.461 63.604) (end 116.565 63.604) (width 1.3) (layer "B.Cu") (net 2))
 (segment (start 114.1625 79.5125) (end 119.105 74.57) (width 1.3) (layer "B.Cu") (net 2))
 (segment (start 109.3 109.22) (end 109.3 108.865) (width 0.3) (layer "B.Cu") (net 2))
 (segment (start 109.3 108.3675) (end 114.1625 103.505) (width 1.3) (layer "B.Cu") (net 2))
 (segment (start 159.745 121.72) (end 159.745 109.22) (width 0.3) (layer "B.Cu") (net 2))
 (segment (start 146.379 123.594) (end 157.871 123.594) (width 0.3) (layer "B.Cu") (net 2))
 (segment (start 114.1625 103.505) (end 114.1625 79.5125) (width 1.3) (layer "B.Cu") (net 2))
 (segment (start 119.105 72.245787) (end 119.105 73.66) (width 1.3) (layer "B.Cu") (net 2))
 (segment (start 134.62 71.12) (end 120.230787 71.12) (width 1.3) (layer "B.Cu") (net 2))
 (segment (start 119.105 74.57) (end 119.105 73.66) (width 1.3) (layer "B.Cu") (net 2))
 (segment (start 119.105 100.605) (end 119.105 99.06) (width 1.3) (layer "B.Cu") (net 2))
 (segment (start 122.666 123.594) (end 124.54 121.72) (width 0.3) (layer "B.Cu") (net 2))
 (segment (start 115.6315 102.036) (end 117.674 102.036) (width 1.3) (layer "B.Cu") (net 2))
 (segment (start 114.1625 103.505) (end 115.6315 102.036) (width 1.3) (layer "B.Cu") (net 2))
 (segment (start 116.84 104.14) (end 119.105 104.14) (width 0.9) (layer "B.Cu") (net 13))
 (segment (start 119.105 104.14) (end 124.185 99.06) (width 0.9) (layer "B.Cu") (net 13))
 (segment (start 118.11 109.22) (end 126.725 100.605) (width 0.9) (layer "B.Cu") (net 3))
 (segment (start 126.725 100.605) (end 126.725 99.06) (width 0.9) (layer "B.Cu") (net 3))
 (segment (start 114.3 109.22) (end 118.11 109.22) (width 0.9) (layer "B.Cu") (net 3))
 (segment (start 114.3 121.72) (end 114.3 109.22) (width 0.3) (layer "B.Cu") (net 3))
 (segment (start 129.54 109.22) (end 129.54 99.335) (width 0.9) (layer "B.Cu") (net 1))
 (segment (start 129.54 99.335) (end 129.265 99.06) (width 0.9) (layer "B.Cu") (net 1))
 (segment (start 129.54 121.72) (end 129.54 109.22) (width 0.3) (layer "B.Cu") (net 1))
 (segment (start 136.525 109.22) (end 131.805 104.5) (width 0.9) (layer "B.Cu") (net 14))
 (segment (start 131.805 104.5) (end 131.805 99.06) (width 0.9) (layer "B.Cu") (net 14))
 (segment (start 139.505 121.72) (end 139.505 109.22) (width 0.3) (layer "B.Cu") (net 14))
 (segment (start 139.505 109.22) (end 136.525 109.22) (width 0.9) (layer "B.Cu") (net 14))
 (segment (start 151.57 106.045) (end 141.33 106.045) (width 0.9) (layer "B.Cu") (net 6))
 (segment (start 154.745 109.22) (end 151.57 106.045) (width 0.9) (layer "B.Cu") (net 6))
 (segment (start 154.745 121.72) (end 154.745 109.22) (width 0.3) (layer "B.Cu") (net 6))
 (segment (start 141.33 106.045) (end 134.345 99.06) (width 0.9) (layer "B.Cu") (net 6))
 (segment (start 157.741396 95.72) (end 145.305 95.72) (width 0.9) (layer "B.Cu") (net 9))
 (segment (start 158.005 95.456396) (end 157.741396 95.72) (width 0.9) (layer "B.Cu") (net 9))
 (segment (start 145.305 95.72) (end 141.965 99.06) (width 0.9) (layer "B.Cu") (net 9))
 (segment (start 158.005 93.98) (end 158.005 95.456396) (width 0.9) (layer "B.Cu") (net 9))
 (segment (start 164.825 93.98) (end 158.005 93.98) (width 0.9) (layer "B.Cu") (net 9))
 (segment (start 164.825 96.52) (end 160.505 100.84) (width 0.9) (layer "B.Cu") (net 10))
 (segment (start 164.825 96.52) (end 164.745 96.44) (width 0.9) (layer "B.Cu") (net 10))
 (segment (start 151.365 100.84) (end 149.585 99.06) (width 0.9) (layer "B.Cu") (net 10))
 (segment (start 160.505 100.84) (end 151.365 100.84) (width 0.9) (layer "B.Cu") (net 10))
 (segment (start 164.825 99.06) (end 166.579 97.306) (width 1.3) (layer "B.Cu") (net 11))
 (segment (start 166.579 97.306) (end 166.579 70.059) (width 1.3) (layer "B.Cu") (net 11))
 (segment (start 166.025 97.86) (end 164.825 99.06) (width 0.3) (layer "B.Cu") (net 11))
 (segment (start 166.579 70.059) (end 153.67 57.15) (width 1.3) (layer "B.Cu") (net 11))
 (segment (start 135.605 63.5) (end 135.605 57.435) (width 1.3) (layer "B.Cu") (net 11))
 (segment (start 135.605 57.435) (end 135.89 57.15) (width 1.3) (layer "B.Cu") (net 11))
 (segment (start 135.89 57.15) (end 153.67 57.15) (width 1.3) (layer "B.Cu") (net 11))
 (segment (start 121.645 63.5) (end 128.005 63.5) (width 0.9) (layer "B.Cu") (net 8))
 (segment (start 109.889 62.196) (end 104.14 67.945) (width 0.9) (layer "B.Cu") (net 7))
 (segment (start 119.105 66.04) (end 119.105 62.59) (width 0.9) (layer "B.Cu") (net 7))
 (segment (start 104.14 67.945) (end 104.14 104.14) (width 0.9) (layer "B.Cu") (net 7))
 (segment (start 119.105 62.59) (end 118.711 62.196) (width 0.9) (layer "B.Cu") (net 7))
 (segment (start 118.711 62.196) (end 109.889 62.196) (width 0.9) (layer "B.Cu") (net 7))
 (segment (start 147.32 63.5) (end 147.32 65.765) (width 0.9) (layer "B.Cu") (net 4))
 (segment (start 147.32 65.765) (end 139.425 73.66) (width 0.9) (layer "B.Cu") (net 4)))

